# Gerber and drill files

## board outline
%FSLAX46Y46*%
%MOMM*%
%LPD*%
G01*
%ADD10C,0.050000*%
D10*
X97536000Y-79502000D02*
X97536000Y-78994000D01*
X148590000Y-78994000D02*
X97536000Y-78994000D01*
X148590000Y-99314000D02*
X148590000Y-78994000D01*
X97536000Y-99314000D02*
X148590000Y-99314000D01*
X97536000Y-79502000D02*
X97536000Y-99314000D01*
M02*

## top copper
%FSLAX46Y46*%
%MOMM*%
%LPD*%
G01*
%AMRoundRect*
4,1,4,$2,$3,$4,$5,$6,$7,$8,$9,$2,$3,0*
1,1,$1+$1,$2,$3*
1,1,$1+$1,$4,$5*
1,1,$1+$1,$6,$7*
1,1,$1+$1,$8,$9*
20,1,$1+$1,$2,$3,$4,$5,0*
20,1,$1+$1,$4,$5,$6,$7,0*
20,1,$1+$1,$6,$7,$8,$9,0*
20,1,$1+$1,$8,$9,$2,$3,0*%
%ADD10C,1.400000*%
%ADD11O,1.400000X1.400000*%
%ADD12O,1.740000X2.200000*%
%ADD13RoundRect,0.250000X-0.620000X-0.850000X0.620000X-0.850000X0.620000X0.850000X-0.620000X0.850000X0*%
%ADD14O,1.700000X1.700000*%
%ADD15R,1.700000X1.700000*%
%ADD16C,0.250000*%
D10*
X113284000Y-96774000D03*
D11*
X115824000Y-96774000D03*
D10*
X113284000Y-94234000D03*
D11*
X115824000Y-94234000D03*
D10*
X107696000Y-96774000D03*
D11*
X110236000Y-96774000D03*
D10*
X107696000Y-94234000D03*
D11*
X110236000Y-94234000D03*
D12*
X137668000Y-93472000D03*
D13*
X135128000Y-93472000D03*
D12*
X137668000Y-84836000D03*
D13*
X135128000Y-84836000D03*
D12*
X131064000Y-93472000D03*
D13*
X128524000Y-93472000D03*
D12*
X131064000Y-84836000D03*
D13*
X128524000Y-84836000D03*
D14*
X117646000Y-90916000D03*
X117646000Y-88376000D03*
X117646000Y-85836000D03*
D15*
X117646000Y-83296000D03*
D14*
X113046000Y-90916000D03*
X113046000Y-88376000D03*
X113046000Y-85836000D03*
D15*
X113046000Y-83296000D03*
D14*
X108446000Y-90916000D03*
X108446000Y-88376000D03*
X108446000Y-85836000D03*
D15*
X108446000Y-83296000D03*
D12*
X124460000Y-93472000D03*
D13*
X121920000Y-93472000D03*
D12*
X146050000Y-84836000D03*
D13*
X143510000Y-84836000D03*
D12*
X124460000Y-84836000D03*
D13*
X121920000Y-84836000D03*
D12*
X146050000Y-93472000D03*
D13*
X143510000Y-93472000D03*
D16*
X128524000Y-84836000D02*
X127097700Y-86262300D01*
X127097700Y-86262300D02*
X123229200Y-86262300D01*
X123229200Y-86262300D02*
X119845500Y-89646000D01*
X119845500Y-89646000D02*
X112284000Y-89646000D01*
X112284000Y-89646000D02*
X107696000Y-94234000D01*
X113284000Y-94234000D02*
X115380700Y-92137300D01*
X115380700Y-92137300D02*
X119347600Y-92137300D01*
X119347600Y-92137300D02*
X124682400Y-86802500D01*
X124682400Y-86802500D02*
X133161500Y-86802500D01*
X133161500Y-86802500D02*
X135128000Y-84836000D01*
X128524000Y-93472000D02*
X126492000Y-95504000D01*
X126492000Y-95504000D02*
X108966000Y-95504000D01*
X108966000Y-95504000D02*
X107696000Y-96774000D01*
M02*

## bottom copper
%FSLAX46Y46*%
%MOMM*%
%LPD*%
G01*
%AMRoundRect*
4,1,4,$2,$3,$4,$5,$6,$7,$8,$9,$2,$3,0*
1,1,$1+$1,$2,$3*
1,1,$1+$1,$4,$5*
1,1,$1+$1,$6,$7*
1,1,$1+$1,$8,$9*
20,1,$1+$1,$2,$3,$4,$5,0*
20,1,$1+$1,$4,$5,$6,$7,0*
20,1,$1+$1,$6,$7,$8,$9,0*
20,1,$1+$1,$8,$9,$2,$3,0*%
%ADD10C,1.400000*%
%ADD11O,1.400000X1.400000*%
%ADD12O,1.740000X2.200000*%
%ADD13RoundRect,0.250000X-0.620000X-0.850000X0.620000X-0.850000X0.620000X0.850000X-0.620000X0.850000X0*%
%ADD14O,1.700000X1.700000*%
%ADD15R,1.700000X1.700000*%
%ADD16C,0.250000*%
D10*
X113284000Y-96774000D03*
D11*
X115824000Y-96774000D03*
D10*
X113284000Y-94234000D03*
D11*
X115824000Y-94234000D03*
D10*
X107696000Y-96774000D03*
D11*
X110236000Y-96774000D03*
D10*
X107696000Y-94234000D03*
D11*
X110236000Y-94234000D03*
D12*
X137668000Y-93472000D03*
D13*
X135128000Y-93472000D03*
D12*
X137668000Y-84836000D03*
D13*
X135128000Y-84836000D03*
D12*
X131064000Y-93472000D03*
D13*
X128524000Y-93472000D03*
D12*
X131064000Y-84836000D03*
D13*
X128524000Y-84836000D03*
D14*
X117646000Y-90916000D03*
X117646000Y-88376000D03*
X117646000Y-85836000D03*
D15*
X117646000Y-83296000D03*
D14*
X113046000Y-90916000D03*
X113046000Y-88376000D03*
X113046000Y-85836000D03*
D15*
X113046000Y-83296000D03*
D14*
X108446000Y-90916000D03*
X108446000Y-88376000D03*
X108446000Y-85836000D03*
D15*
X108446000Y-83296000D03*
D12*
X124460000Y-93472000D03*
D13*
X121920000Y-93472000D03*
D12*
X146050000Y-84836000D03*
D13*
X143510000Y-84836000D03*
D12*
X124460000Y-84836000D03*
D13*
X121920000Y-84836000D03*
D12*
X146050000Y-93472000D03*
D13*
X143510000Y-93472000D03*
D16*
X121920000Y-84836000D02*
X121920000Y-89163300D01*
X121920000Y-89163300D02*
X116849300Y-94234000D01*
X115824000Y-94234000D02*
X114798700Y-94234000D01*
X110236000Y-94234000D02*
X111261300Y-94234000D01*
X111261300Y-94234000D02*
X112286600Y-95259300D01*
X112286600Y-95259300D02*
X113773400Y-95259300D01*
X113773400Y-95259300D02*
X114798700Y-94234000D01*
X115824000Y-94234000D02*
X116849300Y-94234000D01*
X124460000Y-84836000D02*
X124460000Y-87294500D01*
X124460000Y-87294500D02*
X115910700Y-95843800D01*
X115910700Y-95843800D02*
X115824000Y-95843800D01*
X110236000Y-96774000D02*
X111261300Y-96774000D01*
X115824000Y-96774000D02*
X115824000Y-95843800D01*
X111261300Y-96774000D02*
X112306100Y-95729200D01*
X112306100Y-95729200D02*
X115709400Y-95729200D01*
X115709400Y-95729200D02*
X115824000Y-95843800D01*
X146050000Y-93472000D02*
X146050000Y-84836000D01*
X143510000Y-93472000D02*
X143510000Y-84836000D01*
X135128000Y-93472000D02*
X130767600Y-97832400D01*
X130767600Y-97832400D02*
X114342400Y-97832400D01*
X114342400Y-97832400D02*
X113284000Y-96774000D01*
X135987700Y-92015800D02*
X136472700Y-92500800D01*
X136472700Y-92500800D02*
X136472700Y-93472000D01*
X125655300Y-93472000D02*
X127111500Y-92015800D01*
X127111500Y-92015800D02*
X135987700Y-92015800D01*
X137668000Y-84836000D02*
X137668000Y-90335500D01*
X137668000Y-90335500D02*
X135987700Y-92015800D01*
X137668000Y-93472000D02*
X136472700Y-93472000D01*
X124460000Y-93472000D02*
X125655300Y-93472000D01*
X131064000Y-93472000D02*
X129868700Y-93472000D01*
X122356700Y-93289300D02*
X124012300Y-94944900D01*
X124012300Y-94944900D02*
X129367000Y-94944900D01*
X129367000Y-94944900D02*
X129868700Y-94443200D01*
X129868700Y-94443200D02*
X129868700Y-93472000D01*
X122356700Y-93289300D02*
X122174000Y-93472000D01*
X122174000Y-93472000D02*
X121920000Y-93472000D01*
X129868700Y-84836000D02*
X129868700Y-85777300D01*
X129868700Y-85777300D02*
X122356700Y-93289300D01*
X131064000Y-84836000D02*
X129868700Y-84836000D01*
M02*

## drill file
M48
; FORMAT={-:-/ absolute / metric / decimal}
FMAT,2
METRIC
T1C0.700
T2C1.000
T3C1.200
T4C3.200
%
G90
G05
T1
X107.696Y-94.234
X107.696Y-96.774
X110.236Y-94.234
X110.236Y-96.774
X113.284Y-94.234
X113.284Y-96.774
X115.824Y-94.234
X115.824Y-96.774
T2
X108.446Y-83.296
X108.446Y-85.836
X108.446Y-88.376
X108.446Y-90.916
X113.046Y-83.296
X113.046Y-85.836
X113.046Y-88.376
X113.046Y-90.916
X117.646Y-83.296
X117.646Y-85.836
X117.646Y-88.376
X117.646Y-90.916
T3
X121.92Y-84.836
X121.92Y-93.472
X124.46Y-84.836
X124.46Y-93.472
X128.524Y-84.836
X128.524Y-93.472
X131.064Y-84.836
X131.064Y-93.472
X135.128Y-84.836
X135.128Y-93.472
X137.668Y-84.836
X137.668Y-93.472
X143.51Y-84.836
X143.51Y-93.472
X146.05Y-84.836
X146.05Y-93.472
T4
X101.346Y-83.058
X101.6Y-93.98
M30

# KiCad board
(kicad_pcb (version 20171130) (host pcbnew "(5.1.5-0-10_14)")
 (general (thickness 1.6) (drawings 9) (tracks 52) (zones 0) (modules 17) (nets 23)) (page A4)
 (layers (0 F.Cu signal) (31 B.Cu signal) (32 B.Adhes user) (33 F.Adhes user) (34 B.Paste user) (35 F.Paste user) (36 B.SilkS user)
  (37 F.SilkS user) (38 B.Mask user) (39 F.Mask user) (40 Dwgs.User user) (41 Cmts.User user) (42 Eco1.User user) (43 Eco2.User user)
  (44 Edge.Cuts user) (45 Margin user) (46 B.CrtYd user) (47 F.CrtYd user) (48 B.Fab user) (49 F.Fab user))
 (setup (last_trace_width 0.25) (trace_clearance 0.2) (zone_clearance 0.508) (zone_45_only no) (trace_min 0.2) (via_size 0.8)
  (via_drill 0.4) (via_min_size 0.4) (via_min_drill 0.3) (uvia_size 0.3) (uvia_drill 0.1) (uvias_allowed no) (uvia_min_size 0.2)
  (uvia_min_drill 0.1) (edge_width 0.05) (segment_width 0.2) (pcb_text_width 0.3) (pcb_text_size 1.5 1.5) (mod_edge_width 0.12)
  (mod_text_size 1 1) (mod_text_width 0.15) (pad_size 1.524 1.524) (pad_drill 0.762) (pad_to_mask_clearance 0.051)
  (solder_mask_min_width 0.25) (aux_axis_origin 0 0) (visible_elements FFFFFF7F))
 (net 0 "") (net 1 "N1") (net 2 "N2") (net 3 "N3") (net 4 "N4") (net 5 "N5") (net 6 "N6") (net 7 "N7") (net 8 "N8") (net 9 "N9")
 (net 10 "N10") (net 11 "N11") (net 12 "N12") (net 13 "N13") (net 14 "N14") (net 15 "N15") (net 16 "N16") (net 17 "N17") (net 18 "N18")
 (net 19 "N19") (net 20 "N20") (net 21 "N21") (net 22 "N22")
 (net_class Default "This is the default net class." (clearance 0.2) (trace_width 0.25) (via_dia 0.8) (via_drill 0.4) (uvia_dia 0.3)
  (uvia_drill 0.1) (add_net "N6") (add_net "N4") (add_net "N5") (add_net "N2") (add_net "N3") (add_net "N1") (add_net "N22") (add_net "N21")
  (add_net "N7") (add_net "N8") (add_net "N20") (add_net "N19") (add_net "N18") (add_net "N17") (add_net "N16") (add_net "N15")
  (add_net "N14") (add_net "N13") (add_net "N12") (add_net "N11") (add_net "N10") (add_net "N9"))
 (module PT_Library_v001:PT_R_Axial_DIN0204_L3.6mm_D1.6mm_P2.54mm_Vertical (layer F.Cu) (at 113.284 96.774)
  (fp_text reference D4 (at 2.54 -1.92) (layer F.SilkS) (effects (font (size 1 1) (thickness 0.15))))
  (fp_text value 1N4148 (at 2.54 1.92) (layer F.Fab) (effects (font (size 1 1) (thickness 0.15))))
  (pad 1 thru_hole circle (at 0 0) (size 1.4 1.4) (drill 0.7) (layers *.Cu *.Mask) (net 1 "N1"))
  (pad 2 thru_hole oval (at 2.54 0) (size 1.4 1.4) (drill 0.7) (layers *.Cu *.Mask) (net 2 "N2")))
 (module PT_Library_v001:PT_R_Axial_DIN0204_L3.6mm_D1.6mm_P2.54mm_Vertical (layer F.Cu) (at 113.284 94.234)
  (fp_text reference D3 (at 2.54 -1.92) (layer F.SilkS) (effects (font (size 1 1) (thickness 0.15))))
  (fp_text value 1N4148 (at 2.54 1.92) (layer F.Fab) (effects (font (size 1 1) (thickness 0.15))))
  (pad 1 thru_hole circle (at 0 0) (size 1.4 1.4) (drill 0.7) (layers *.Cu *.Mask) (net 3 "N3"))
  (pad 2 thru_hole oval (at 2.54 0) (size 1.4 1.4) (drill 0.7) (layers *.Cu *.Mask) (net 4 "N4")))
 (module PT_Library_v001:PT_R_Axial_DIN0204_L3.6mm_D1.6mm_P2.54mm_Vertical (layer F.Cu) (at 107.696 96.774)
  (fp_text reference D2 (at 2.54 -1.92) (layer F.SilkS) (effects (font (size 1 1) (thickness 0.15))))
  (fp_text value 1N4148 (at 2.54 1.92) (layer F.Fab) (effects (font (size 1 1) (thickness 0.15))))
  (pad 1 thru_hole circle (at 0 0) (size 1.4 1.4) (drill 0.7) (layers *.Cu *.Mask) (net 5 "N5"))
  (pad 2 thru_hole oval (at 2.54 0) (size 1.4 1.4) (drill 0.7) (layers *.Cu *.Mask) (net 2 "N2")))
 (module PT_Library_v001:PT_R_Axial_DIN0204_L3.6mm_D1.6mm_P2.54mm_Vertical (layer F.Cu) (at 107.696 94.234)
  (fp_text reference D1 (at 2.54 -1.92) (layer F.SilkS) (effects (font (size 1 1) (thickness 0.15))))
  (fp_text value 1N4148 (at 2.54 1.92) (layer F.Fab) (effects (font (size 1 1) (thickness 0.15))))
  (pad 1 thru_hole circle (at 0 0) (size 1.4 1.4) (drill 0.7) (layers *.Cu *.Mask) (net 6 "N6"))
  (pad 2 thru_hole oval (at 2.54 0) (size 1.4 1.4) (drill 0.7) (layers *.Cu *.Mask) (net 4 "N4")))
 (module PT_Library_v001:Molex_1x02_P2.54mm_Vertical (layer F.Cu) (at 135.128 93.472)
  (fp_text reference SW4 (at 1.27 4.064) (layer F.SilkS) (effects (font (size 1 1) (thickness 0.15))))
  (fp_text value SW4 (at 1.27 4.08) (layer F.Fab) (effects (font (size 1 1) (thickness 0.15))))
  (pad 2 thru_hole oval (at 2.54 0) (size 1.74 2.2) (drill 1.2) (layers *.Cu *.Mask) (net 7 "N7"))
  (pad 1 thru_hole roundrect (at 0 0) (size 1.74 2.2) (drill 1.2) (layers *.Cu *.Mask) (roundrect_rratio 0.143678) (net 1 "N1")))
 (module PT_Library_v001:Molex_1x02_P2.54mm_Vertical (layer F.Cu) (at 135.128 84.836)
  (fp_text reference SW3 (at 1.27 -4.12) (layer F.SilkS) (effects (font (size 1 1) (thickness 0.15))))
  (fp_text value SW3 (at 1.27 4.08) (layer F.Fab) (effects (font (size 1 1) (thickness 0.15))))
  (pad 2 thru_hole oval (at 2.54 0) (size 1.74 2.2) (drill 1.2) (layers *.Cu *.Mask) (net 7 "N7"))
  (pad 1 thru_hole roundrect (at 0 0) (size 1.74 2.2) (drill 1.2) (layers *.Cu *.Mask) (roundrect_rratio 0.143678) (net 3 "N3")))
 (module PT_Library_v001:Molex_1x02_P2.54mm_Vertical (layer F.Cu) (at 128.524 93.472)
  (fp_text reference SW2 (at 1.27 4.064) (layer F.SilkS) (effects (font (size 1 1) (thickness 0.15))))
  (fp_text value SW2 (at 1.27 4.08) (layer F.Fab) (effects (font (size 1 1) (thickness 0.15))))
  (pad 2 thru_hole oval (at 2.54 0) (size 1.74 2.2) (drill 1.2) (layers *.Cu *.Mask) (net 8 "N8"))
  (pad 1 thru_hole roundrect (at 0 0) (size 1.74 2.2) (drill 1.2) (layers *.Cu *.Mask) (roundrect_rratio 0.143678) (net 5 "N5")))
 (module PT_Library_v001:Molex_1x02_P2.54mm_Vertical (layer F.Cu) (at 128.524 84.836)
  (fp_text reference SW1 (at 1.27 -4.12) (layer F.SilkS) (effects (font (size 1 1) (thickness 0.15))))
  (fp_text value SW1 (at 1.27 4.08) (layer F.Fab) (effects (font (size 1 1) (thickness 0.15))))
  (pad 2 thru_hole oval (at 2.54 0) (size 1.74 2.2) (drill 1.2) (layers *.Cu *.Mask) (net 8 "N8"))
  (pad 1 thru_hole roundrect (at 0 0) (size 1.74 2.2) (drill 1.2) (layers *.Cu *.Mask) (roundrect_rratio 0.143678) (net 6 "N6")))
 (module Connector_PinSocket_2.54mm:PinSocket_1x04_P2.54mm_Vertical (layer F.Cu) (at 117.646 83.296)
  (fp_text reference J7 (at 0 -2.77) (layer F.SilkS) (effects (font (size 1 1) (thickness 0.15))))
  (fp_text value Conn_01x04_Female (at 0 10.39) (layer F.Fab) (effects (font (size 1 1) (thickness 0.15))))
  (pad 4 thru_hole oval (at 0 7.62) (size 1.7 1.7) (drill 1) (layers *.Cu *.Mask) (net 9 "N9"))
  (pad 3 thru_hole oval (at 0 5.08) (size 1.7 1.7) (drill 1) (layers *.Cu *.Mask) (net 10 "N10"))
  (pad 2 thru_hole oval (at 0 2.54) (size 1.7 1.7) (drill 1) (layers *.Cu *.Mask) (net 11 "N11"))
  (pad 1 thru_hole rect (at 0 0) (size 1.7 1.7) (drill 1) (layers *.Cu *.Mask) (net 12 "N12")))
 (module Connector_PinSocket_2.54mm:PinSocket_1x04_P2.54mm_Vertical (layer F.Cu) (at 113.046 83.296)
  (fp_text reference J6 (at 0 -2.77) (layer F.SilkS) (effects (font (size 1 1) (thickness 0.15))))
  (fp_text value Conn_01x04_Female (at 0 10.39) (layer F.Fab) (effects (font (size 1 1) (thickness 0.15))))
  (pad 4 thru_hole oval (at 0 7.62) (size 1.7 1.7) (drill 1) (layers *.Cu *.Mask) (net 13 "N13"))
  (pad 3 thru_hole oval (at 0 5.08) (size 1.7 1.7) (drill 1) (layers *.Cu *.Mask) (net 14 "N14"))
  (pad 2 thru_hole oval (at 0 2.54) (size 1.7 1.7) (drill 1) (layers *.Cu *.Mask) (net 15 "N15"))
  (pad 1 thru_hole rect (at 0 0) (size 1.7 1.7) (drill 1) (layers *.Cu *.Mask) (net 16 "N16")))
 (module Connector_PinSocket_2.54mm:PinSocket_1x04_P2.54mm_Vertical (layer F.Cu) (at 108.446 83.296)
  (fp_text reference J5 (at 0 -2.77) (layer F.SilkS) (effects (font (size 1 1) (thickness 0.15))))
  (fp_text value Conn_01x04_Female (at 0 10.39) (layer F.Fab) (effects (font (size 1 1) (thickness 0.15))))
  (pad 4 thru_hole oval (at 0 7.62) (size 1.7 1.7) (drill 1) (layers *.Cu *.Mask) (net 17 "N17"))
  (pad 3 thru_hole oval (at 0 5.08) (size 1.7 1.7) (drill 1) (layers *.Cu *.Mask) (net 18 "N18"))
  (pad 2 thru_hole oval (at 0 2.54) (size 1.7 1.7) (drill 1) (layers *.Cu *.Mask) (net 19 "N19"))
  (pad 1 thru_hole rect (at 0 0) (size 1.7 1.7) (drill 1) (layers *.Cu *.Mask) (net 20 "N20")))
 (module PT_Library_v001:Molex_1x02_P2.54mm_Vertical (layer F.Cu) (at 121.92 93.472)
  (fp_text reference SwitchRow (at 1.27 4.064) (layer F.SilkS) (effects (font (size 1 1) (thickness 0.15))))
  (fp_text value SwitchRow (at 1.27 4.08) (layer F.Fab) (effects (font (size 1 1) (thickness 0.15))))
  (pad 2 thru_hole oval (at 2.54 0) (size 1.74 2.2) (drill 1.2) (layers *.Cu *.Mask) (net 7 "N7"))
  (pad 1 thru_hole roundrect (at 0 0) (size 1.74 2.2) (drill 1.2) (layers *.Cu *.Mask) (roundrect_rratio 0.143678) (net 8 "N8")))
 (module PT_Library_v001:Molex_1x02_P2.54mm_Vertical (layer F.Cu) (at 143.51 84.836)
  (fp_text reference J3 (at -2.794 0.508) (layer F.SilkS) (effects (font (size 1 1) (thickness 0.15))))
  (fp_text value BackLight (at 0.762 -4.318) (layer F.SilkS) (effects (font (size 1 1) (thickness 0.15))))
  (pad 2 thru_hole oval (at 2.54 0) (size 1.74 2.2) (drill 1.2) (layers *.Cu *.Mask) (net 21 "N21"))
  (pad 1 thru_hole roundrect (at 0 0) (size 1.74 2.2) (drill 1.2) (layers *.Cu *.Mask) (roundrect_rratio 0.143678) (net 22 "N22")))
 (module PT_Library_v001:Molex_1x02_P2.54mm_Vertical (layer F.Cu) (at 121.92 84.836)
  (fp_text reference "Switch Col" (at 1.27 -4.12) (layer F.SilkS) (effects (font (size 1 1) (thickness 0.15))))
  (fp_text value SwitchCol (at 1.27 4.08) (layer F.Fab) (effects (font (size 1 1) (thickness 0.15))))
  (pad 2 thru_hole oval (at 2.54 0) (size 1.74 2.2) (drill 1.2) (layers *.Cu *.Mask) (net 2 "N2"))
  (pad 1 thru_hole roundrect (at 0 0) (size 1.74 2.2) (drill 1.2) (layers *.Cu *.Mask) (roundrect_rratio 0.143678) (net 4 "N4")))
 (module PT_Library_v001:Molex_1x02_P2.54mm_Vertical (layer F.Cu) (at 143.51 93.472)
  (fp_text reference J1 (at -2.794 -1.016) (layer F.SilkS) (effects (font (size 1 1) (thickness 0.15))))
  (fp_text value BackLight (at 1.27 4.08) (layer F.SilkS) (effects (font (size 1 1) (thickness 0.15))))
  (pad 2 thru_hole oval (at 2.54 0) (size 1.74 2.2) (drill 1.2) (layers *.Cu *.Mask) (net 21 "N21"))
  (pad 1 thru_hole roundrect (at 0 0) (size 1.74 2.2) (drill 1.2) (layers *.Cu *.Mask) (roundrect_rratio 0.143678) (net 22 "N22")))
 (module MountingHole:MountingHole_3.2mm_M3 (layer F.Cu) (at 101.346 83.058)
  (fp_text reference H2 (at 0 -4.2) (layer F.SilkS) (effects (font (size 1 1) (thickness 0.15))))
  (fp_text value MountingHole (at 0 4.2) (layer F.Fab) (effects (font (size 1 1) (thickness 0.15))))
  (pad 1 np_thru_hole circle (at 0 0) (size 3.2 3.2) (drill 3.2) (layers *.Cu *.Mask)))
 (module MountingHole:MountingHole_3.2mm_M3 (layer F.Cu) (at 101.6 93.98)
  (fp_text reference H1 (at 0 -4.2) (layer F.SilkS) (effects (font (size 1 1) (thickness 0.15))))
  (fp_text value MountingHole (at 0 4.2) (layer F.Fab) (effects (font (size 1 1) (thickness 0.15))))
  (pad 1 np_thru_hole circle (at 0 0) (size 3.2 3.2) (drill 3.2) (layers *.Cu *.Mask)))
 (gr_line (start 97.536 79.502) (end 97.536 78.994) (layer Edge.Cuts) (width 0.05))
 (gr_line (start 148.59 78.994) (end 97.536 78.994) (layer Edge.Cuts) (width 0.05))
 (gr_line (start 148.59 99.314) (end 148.59 78.994) (layer Edge.Cuts) (width 0.05))
 (gr_line (start 97.536 99.314) (end 148.59 99.314) (layer Edge.Cuts) (width 0.05))
 (gr_line (start 97.536 79.502) (end 97.536 99.314) (layer Edge.Cuts) (width 0.05))
 (segment (start 121.92 84.836) (end 121.92 89.1633) (width 0.25) (layer B.Cu) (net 4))
 (segment (start 121.92 89.1633) (end 116.8493 94.234) (width 0.25) (layer B.Cu) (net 4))
 (segment (start 115.824 94.234) (end 114.7987 94.234) (width 0.25) (layer B.Cu) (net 4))
 (segment (start 110.236 94.234) (end 111.2613 94.234) (width 0.25) (layer B.Cu) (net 4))
 (segment (start 111.2613 94.234) (end 112.2866 95.2593) (width 0.25) (layer B.Cu) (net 4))
 (segment (start 112.2866 95.2593) (end 113.7734 95.2593) (width 0.25) (layer B.Cu) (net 4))
 (segment (start 113.7734 95.2593) (end 114.7987 94.234) (width 0.25) (layer B.Cu) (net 4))
 (segment (start 115.824 94.234) (end 116.8493 94.234) (width 0.25) (layer B.Cu) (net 4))
 (segment (start 128.524 84.836) (end 127.0977 86.2623) (width 0.25) (layer F.Cu) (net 6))
 (segment (start 127.0977 86.2623) (end 123.2292 86.2623) (width 0.25) (layer F.Cu) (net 6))
 (segment (start 123.2292 86.2623) (end 119.8455 89.646) (width 0.25) (layer F.Cu) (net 6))
 (segment (start 119.8455 89.646) (end 112.284 89.646) (width 0.25) (layer F.Cu) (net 6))
 (segment (start 112.284 89.646) (end 107.696 94.234) (width 0.25) (layer F.Cu) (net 6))
 (segment (start 124.46 84.836) (end 124.46 87.2945) (width 0.25) (layer B.Cu) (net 2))
 (segment (start 124.46 87.2945) (end 115.9107 95.8438) (width 0.25) (layer B.Cu) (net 2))
 (segment (start 115.9107 95.8438) (end 115.824 95.8438) (width 0.25) (layer B.Cu) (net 2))
 (segment (start 110.236 96.774) (end 111.2613 96.774) (width 0.25) (layer B.Cu) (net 2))
 (segment (start 115.824 96.774) (end 115.824 95.8438) (width 0.25) (layer B.Cu) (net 2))
 (segment (start 111.2613 96.774) (end 112.3061 95.7292) (width 0.25) (layer B.Cu) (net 2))
 (segment (start 112.3061 95.7292) (end 115.7094 95.7292) (width 0.25) (layer B.Cu) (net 2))
 (segment (start 115.7094 95.7292) (end 115.824 95.8438) (width 0.25) (layer B.Cu) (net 2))
 (segment (start 113.284 94.234) (end 115.3807 92.1373) (width 0.25) (layer F.Cu) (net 3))
 (segment (start 115.3807 92.1373) (end 119.3476 92.1373) (width 0.25) (layer F.Cu) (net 3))
 (segment (start 119.3476 92.1373) (end 124.6824 86.8025) (width 0.25) (layer F.Cu) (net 3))
 (segment (start 124.6824 86.8025) (end 133.1615 86.8025) (width 0.25) (layer F.Cu) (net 3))
 (segment (start 133.1615 86.8025) (end 135.128 84.836) (width 0.25) (layer F.Cu) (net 3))
 (segment (start 146.05 93.472) (end 146.05 84.836) (width 0.25) (layer B.Cu) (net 21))
 (segment (start 143.51 93.472) (end 143.51 84.836) (width 0.25) (layer B.Cu) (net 22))
 (segment (start 128.524 93.472) (end 126.492 95.504) (width 0.25) (layer F.Cu) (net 5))
 (segment (start 126.492 95.504) (end 108.966 95.504) (width 0.25) (layer F.Cu) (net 5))
 (segment (start 108.966 95.504) (end 107.696 96.774) (width 0.25) (layer F.Cu) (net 5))
 (segment (start 135.128 93.472) (end 130.7676 97.8324) (width 0.25) (layer B.Cu) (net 1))
 (segment (start 130.7676 97.8324) (end 114.3424 97.8324) (width 0.25) (layer B.Cu) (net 1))
 (segment (start 114.3424 97.8324) (end 113.284 96.774) (width 0.25) (layer B.Cu) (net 1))
 (segment (start 135.9877 92.0158) (end 136.4727 92.5008) (width 0.25) (layer B.Cu) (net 7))
 (segment (start 136.4727 92.5008) (end 136.4727 93.472) (width 0.25) (layer B.Cu) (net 7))
 (segment (start 125.6553 93.472) (end 127.1115 92.0158) (width 0.25) (layer B.Cu) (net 7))
 (segment (start 127.1115 92.0158) (end 135.9877 92.0158) (width 0.25) (layer B.Cu) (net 7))
 (segment (start 137.668 84.836) (end 137.668 90.3355) (width 0.25) (layer B.Cu) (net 7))
 (segment (start 137.668 90.3355) (end 135.9877 92.0158) (width 0.25) (layer B.Cu) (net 7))
 (segment (start 137.668 93.472) (end 136.4727 93.472) (width 0.25) (layer B.Cu) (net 7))
 (segment (start 124.46 93.472) (end 125.6553 93.472) (width 0.25) (layer B.Cu) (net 7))
 (segment (start 131.064 93.472) (end 129.8687 93.472) (width 0.25) (layer B.Cu) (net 8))
 (segment (start 122.3567 93.2893) (end 124.0123 94.9449) (width 0.25) (layer B.Cu) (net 8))
 (segment (start 124.0123 94.9449) (end 129.367 94.9449) (width 0.25) (layer B.Cu) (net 8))
 (segment (start 129.367 94.9449) (end 129.8687 94.4432) (width 0.25) (layer B.Cu) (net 8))
 (segment (start 129.8687 94.4432) (end 129.8687 93.472) (width 0.25) (layer B.Cu) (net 8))
 (segment (start 122.3567 93.2893) (end 122.174 93.472) (width 0.25) (layer B.Cu) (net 8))
 (segment (start 122.174 93.472) (end 121.92 93.472) (width 0.25) (layer B.Cu) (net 8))
 (segment (start 129.8687 84.836) (end 129.8687 85.7773) (width 0.25) (layer B.Cu) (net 8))
 (segment (start 129.8687 85.7773) (end 122.3567 93.2893) (width 0.25) (layer B.Cu) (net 8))
 (segment (start 131.064 84.836) (end 129.8687 84.836) (width 0.25) (layer B.Cu) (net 8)))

